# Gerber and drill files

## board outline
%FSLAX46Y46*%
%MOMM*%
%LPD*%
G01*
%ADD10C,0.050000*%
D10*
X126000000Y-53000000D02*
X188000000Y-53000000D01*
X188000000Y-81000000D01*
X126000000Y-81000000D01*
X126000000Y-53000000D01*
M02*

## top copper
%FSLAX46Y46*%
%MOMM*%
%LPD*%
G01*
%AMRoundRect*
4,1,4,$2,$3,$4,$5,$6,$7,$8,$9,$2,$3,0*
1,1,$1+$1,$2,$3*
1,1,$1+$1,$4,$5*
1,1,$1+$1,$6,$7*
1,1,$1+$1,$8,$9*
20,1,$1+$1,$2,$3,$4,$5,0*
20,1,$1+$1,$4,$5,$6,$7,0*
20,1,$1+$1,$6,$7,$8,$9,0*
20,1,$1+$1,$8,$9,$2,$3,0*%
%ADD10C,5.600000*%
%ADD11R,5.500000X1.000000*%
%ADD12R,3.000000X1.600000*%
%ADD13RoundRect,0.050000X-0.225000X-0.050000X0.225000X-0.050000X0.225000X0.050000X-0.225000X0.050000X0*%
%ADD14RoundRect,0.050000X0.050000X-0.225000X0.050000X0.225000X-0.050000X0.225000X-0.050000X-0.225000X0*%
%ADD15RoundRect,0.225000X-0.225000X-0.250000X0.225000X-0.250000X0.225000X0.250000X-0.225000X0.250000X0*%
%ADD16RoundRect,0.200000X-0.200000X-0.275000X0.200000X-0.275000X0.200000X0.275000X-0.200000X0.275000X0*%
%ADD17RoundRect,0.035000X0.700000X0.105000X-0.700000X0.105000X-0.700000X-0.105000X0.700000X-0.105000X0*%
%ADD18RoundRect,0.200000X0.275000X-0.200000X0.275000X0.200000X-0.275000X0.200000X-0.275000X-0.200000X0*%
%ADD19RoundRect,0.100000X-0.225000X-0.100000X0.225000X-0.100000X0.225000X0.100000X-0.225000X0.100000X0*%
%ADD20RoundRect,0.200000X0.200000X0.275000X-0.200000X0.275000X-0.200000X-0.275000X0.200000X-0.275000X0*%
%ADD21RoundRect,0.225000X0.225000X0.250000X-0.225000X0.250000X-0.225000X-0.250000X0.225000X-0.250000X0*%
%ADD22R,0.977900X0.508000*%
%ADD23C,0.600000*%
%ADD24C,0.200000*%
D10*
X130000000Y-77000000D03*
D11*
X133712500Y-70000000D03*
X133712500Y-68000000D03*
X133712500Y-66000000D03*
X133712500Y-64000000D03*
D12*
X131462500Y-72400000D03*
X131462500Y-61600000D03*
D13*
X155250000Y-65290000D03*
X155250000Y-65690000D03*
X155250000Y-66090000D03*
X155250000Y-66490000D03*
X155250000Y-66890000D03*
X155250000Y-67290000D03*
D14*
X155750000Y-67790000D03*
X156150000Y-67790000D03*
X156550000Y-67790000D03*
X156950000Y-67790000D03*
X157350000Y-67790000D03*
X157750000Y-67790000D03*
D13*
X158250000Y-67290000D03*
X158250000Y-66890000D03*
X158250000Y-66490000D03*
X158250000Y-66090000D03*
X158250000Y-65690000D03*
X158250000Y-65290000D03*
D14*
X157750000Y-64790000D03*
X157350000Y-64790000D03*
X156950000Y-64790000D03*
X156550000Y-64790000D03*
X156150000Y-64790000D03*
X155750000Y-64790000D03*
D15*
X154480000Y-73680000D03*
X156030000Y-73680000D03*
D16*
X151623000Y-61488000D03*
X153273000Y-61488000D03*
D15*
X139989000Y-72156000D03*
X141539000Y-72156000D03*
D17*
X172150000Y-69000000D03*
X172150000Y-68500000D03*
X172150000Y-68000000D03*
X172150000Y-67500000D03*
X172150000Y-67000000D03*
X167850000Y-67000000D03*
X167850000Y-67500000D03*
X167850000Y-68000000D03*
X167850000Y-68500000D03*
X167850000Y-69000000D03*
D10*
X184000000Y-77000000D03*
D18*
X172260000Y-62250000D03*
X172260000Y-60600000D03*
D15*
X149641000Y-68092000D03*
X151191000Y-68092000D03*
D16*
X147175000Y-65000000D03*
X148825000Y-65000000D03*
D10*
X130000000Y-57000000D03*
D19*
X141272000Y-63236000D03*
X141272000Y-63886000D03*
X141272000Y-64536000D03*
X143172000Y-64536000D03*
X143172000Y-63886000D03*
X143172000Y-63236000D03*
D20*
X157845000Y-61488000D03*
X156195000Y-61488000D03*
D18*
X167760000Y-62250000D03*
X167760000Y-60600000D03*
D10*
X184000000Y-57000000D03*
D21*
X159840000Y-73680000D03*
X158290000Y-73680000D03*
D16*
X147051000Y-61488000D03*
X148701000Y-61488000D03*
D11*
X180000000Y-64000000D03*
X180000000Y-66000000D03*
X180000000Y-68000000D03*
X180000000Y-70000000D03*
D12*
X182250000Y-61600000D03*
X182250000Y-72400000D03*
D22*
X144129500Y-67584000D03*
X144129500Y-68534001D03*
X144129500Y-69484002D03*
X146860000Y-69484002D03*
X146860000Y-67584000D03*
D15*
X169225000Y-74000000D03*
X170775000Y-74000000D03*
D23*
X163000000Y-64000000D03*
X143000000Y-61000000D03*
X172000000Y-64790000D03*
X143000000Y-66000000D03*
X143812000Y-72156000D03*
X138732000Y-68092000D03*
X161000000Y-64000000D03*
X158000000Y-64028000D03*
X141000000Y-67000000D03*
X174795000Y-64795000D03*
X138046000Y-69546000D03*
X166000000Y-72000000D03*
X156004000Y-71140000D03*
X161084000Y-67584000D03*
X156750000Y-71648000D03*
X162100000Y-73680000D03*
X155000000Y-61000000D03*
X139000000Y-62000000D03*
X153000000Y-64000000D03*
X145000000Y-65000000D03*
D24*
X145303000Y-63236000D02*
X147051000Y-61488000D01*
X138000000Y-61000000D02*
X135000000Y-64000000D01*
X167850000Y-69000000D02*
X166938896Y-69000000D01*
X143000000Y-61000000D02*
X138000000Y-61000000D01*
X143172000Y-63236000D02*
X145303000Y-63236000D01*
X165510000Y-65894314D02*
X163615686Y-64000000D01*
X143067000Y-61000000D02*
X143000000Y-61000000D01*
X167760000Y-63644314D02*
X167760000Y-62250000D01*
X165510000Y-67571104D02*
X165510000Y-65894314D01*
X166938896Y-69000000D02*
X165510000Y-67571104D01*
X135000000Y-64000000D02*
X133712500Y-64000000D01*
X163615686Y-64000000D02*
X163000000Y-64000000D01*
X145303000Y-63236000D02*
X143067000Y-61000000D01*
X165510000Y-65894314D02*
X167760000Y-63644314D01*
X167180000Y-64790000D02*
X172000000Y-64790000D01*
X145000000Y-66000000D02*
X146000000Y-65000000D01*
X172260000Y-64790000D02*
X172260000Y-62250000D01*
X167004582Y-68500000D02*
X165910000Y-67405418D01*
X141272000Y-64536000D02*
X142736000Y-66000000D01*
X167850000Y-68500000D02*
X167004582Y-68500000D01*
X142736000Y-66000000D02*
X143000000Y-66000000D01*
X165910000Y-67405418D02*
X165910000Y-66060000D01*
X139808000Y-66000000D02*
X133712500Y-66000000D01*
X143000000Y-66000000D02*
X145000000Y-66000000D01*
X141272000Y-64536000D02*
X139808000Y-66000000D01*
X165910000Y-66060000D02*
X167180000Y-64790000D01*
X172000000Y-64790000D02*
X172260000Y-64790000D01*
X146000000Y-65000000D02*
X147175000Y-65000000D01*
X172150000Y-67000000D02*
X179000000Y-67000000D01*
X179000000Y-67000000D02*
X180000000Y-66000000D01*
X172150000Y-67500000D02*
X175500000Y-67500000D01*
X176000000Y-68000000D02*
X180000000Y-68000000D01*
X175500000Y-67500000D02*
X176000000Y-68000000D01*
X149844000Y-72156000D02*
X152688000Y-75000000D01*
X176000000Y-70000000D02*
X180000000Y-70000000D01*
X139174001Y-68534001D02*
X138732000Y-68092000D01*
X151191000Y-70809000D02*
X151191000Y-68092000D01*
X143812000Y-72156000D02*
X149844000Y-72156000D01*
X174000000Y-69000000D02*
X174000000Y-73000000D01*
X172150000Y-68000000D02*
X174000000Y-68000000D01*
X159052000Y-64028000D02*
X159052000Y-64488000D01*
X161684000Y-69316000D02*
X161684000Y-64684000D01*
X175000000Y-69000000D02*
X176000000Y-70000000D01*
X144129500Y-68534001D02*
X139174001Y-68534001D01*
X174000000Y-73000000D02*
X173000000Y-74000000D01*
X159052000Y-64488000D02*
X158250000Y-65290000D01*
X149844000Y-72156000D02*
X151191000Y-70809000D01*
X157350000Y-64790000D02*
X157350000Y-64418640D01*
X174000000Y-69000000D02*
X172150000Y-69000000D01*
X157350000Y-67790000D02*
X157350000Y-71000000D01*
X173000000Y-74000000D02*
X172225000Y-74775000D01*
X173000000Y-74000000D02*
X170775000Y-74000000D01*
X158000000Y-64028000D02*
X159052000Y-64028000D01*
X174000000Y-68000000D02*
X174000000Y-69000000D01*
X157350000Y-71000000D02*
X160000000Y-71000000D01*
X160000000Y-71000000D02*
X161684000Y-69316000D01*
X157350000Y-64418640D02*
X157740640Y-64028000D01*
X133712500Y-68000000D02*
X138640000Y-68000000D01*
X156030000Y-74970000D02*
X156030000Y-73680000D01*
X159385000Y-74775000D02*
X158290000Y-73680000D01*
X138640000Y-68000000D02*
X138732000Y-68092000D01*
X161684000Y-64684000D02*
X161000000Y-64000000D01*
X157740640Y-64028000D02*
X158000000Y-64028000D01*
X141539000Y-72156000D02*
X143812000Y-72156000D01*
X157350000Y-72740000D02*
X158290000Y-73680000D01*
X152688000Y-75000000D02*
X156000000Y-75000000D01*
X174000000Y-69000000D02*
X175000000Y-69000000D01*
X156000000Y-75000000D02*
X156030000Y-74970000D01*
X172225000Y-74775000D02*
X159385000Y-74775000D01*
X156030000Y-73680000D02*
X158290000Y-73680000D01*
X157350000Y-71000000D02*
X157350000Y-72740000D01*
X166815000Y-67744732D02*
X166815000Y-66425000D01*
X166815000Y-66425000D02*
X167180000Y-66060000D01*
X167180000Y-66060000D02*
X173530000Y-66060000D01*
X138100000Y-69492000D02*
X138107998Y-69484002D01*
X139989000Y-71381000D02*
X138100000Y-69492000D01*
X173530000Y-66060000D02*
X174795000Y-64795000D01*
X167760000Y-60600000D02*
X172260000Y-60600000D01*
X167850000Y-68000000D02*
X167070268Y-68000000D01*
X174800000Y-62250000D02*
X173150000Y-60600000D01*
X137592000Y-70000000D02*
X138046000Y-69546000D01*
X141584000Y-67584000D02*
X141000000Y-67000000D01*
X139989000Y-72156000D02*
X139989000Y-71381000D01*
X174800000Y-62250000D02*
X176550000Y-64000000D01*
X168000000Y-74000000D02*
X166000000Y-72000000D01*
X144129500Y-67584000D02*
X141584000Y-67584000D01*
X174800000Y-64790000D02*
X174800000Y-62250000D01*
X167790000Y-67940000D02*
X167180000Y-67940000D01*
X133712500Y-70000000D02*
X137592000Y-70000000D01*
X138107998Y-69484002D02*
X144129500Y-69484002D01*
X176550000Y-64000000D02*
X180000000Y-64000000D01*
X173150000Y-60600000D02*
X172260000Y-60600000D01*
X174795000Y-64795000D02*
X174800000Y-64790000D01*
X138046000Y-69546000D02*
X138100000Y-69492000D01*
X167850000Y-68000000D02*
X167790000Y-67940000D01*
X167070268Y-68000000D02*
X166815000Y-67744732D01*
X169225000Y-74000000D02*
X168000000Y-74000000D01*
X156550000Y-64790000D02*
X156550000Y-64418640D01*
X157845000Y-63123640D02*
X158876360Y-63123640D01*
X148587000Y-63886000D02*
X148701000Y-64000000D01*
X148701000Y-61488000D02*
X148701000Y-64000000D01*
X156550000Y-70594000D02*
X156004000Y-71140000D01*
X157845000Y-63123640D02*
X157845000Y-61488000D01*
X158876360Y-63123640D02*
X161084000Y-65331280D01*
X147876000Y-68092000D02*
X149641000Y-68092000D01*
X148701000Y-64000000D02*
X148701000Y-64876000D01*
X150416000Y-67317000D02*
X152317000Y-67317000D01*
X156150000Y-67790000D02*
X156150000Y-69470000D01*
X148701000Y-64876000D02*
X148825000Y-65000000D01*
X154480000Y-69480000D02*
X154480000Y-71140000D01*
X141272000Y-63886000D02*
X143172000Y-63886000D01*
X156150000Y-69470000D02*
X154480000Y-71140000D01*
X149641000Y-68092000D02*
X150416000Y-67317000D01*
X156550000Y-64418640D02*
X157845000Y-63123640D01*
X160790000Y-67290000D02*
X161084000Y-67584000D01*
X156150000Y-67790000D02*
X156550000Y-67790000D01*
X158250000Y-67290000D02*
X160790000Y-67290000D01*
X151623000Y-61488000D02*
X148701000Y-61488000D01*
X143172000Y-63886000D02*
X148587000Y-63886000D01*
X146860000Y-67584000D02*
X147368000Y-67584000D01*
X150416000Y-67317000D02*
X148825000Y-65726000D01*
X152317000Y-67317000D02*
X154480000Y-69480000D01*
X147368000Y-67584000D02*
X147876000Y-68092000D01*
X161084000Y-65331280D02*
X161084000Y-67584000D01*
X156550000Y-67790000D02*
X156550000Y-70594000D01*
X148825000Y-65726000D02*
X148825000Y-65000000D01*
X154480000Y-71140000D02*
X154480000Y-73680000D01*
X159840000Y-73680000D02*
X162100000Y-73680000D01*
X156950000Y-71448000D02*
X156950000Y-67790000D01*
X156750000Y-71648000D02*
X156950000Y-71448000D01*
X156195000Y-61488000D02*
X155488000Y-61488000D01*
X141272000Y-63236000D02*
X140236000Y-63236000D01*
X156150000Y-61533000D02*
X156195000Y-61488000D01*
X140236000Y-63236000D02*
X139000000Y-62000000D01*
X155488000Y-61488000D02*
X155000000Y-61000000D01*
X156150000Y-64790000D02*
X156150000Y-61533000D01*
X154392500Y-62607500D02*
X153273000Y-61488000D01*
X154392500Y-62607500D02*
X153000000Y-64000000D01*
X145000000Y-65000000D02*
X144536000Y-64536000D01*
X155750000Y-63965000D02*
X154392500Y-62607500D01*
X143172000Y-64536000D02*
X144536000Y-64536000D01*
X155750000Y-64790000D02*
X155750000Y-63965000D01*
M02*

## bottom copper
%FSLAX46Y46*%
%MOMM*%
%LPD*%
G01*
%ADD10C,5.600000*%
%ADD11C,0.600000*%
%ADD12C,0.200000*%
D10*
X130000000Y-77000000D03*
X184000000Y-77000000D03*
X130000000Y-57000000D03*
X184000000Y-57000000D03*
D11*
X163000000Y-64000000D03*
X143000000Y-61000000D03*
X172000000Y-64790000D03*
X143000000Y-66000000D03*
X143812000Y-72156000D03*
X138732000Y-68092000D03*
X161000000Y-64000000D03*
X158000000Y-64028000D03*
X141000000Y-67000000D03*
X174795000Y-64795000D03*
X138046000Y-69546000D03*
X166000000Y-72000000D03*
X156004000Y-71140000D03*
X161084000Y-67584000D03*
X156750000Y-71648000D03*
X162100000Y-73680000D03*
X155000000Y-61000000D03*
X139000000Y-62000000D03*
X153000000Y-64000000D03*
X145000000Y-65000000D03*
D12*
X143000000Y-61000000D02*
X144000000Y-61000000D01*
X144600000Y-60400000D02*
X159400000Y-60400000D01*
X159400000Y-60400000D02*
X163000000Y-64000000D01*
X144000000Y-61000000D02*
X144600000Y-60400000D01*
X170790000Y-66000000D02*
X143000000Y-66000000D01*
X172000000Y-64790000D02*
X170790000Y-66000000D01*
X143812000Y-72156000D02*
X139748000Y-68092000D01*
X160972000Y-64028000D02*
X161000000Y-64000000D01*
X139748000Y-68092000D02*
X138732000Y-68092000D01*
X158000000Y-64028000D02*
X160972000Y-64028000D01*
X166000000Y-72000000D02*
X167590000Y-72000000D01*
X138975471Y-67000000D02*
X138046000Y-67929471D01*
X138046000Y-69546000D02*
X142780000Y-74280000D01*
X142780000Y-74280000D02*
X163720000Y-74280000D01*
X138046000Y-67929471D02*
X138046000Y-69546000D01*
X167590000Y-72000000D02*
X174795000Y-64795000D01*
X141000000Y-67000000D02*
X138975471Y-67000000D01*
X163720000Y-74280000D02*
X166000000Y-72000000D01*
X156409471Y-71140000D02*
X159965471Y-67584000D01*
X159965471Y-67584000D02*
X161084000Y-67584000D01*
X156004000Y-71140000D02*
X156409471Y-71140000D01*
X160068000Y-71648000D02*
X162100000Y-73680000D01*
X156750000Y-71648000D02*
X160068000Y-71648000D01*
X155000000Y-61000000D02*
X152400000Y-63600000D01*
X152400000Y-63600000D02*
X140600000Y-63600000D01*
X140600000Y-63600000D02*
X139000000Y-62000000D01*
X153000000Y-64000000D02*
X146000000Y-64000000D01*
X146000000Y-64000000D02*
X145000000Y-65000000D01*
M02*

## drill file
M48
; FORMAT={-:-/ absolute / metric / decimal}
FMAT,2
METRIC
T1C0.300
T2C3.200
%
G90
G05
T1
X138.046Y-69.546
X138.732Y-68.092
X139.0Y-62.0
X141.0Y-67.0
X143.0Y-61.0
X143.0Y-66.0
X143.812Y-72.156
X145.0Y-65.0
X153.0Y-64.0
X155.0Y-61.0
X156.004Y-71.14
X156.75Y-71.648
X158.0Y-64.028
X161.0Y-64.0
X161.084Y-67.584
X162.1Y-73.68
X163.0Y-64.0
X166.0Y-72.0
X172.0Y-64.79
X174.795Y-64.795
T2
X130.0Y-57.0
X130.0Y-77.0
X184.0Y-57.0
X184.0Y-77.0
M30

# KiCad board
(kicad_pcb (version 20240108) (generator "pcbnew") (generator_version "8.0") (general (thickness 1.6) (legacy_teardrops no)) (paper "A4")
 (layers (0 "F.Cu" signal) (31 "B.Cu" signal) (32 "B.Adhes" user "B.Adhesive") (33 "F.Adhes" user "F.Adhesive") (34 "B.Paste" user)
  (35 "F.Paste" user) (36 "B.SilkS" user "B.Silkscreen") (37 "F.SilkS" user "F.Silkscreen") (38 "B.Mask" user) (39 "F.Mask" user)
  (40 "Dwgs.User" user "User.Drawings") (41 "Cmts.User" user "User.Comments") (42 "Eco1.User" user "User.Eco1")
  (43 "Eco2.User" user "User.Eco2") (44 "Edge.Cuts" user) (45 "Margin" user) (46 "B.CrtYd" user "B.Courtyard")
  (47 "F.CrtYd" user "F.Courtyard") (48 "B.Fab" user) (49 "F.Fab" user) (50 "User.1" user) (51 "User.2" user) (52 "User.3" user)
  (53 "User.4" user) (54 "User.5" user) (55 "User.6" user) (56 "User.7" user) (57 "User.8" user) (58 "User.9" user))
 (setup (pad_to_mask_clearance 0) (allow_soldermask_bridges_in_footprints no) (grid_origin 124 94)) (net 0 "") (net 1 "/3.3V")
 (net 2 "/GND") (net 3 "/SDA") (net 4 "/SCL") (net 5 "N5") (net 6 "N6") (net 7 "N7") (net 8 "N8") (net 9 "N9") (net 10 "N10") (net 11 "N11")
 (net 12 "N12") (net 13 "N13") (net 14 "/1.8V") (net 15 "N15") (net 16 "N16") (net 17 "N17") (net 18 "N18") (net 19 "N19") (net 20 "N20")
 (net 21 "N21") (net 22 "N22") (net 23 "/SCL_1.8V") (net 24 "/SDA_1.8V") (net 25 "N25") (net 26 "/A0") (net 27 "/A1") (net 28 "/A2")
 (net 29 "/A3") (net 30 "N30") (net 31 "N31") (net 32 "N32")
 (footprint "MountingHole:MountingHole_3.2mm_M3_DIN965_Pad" (layer "F.Cu") (at 130 77)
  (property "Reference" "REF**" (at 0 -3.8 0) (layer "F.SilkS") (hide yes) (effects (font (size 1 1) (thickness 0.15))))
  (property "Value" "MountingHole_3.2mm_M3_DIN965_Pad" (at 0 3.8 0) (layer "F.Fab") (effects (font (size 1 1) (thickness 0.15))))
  (pad "1" thru_hole circle (at 0 0) (size 5.6 5.6) (drill 3.2) (layers "*.Cu" "*.Mask") (remove_unused_layers no)))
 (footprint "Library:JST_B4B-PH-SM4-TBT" (layer "F.Cu") (at 131.4625 67 90)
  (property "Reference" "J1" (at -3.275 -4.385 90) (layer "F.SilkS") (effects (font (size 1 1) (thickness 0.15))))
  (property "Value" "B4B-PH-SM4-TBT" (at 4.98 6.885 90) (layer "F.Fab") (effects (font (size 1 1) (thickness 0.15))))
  (pad "1" smd rect (at -3 2.25 90) (size 1 5.5) (layers "F.Cu" "F.Paste" "F.Mask") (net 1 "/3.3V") (solder_mask_margin 0.102))
  (pad "2" smd rect (at -1 2.25 90) (size 1 5.5) (layers "F.Cu" "F.Paste" "F.Mask") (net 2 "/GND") (solder_mask_margin 0.102))
  (pad "3" smd rect (at 1 2.25 90) (size 1 5.5) (layers "F.Cu" "F.Paste" "F.Mask") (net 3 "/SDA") (solder_mask_margin 0.102))
  (pad "4" smd rect (at 3 2.25 90) (size 1 5.5) (layers "F.Cu" "F.Paste" "F.Mask") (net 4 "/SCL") (solder_mask_margin 0.102))
  (pad "SH1" smd rect (at -5.4 0 90) (size 1.6 3) (layers "F.Cu" "F.Paste" "F.Mask") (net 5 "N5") (solder_mask_margin 0.102))
  (pad "SH2" smd rect (at 5.4 0 90) (size 1.6 3) (layers "F.Cu" "F.Paste" "F.Mask") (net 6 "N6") (solder_mask_margin 0.102)))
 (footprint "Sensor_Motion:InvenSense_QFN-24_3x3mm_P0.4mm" (layer "F.Cu") (at 156.75 66.29)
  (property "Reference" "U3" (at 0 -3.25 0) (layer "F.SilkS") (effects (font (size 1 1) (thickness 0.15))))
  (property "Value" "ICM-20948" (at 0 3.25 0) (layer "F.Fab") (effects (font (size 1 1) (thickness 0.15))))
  (pad "1" smd roundrect (at -1.5 -1) (size 0.55 0.2) (layers "F.Cu" "F.Paste" "F.Mask") (roundrect_rratio 0.25) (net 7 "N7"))
  (pad "2" smd roundrect (at -1.5 -0.6) (size 0.55 0.2) (layers "F.Cu" "F.Paste" "F.Mask") (roundrect_rratio 0.25) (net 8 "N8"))
  (pad "3" smd roundrect (at -1.5 -0.2) (size 0.55 0.2) (layers "F.Cu" "F.Paste" "F.Mask") (roundrect_rratio 0.25) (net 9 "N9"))
  (pad "4" smd roundrect (at -1.5 0.2) (size 0.55 0.2) (layers "F.Cu" "F.Paste" "F.Mask") (roundrect_rratio 0.25) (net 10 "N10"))
  (pad "5" smd roundrect (at -1.5 0.6) (size 0.55 0.2) (layers "F.Cu" "F.Paste" "F.Mask") (roundrect_rratio 0.25) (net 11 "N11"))
  (pad "6" smd roundrect (at -1.5 1) (size 0.55 0.2) (layers "F.Cu" "F.Paste" "F.Mask") (roundrect_rratio 0.25) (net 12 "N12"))
  (pad "7" smd roundrect (at -1 1.5 90) (size 0.55 0.2) (layers "F.Cu" "F.Paste" "F.Mask") (roundrect_rratio 0.25) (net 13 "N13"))
  (pad "8" smd roundrect (at -0.6 1.5 90) (size 0.55 0.2) (layers "F.Cu" "F.Paste" "F.Mask") (roundrect_rratio 0.25) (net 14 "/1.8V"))
  (pad "9" smd roundrect (at -0.2 1.5 90) (size 0.55 0.2) (layers "F.Cu" "F.Paste" "F.Mask") (roundrect_rratio 0.25) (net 14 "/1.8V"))
  (pad "10" smd roundrect (at 0.2 1.5 90) (size 0.55 0.2) (layers "F.Cu" "F.Paste" "F.Mask") (roundrect_rratio 0.25) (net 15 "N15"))
  (pad "11" smd roundrect (at 0.6 1.5 90) (size 0.55 0.2) (layers "F.Cu" "F.Paste" "F.Mask") (roundrect_rratio 0.25) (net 2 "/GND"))
  (pad "12" smd roundrect (at 1 1.5 90) (size 0.55 0.2) (layers "F.Cu" "F.Paste" "F.Mask") (roundrect_rratio 0.25) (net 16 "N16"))
  (pad "13" smd roundrect (at 1.5 1) (size 0.55 0.2) (layers "F.Cu" "F.Paste" "F.Mask") (roundrect_rratio 0.25) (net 14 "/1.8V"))
  (pad "14" smd roundrect (at 1.5 0.6) (size 0.55 0.2) (layers "F.Cu" "F.Paste" "F.Mask") (roundrect_rratio 0.25) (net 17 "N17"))
  (pad "15" smd roundrect (at 1.5 0.2) (size 0.55 0.2) (layers "F.Cu" "F.Paste" "F.Mask") (roundrect_rratio 0.25) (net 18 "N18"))
  (pad "16" smd roundrect (at 1.5 -0.2) (size 0.55 0.2) (layers "F.Cu" "F.Paste" "F.Mask") (roundrect_rratio 0.25) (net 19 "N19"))
  (pad "17" smd roundrect (at 1.5 -0.6) (size 0.55 0.2) (layers "F.Cu" "F.Paste" "F.Mask") (roundrect_rratio 0.25) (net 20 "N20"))
  (pad "18" smd roundrect (at 1.5 -1) (size 0.55 0.2) (layers "F.Cu" "F.Paste" "F.Mask") (roundrect_rratio 0.25) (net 2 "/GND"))
  (pad "19" smd roundrect (at 1 -1.5 90) (size 0.55 0.2) (layers "F.Cu" "F.Paste" "F.Mask") (roundrect_rratio 0.25) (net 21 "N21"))
  (pad "20" smd roundrect (at 0.6 -1.5 90) (size 0.55 0.2) (layers "F.Cu" "F.Paste" "F.Mask") (roundrect_rratio 0.25) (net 2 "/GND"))
  (pad "21" smd roundrect (at 0.2 -1.5 90) (size 0.55 0.2) (layers "F.Cu" "F.Paste" "F.Mask") (roundrect_rratio 0.25) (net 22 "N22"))
  (pad "22" smd roundrect (at -0.2 -1.5 90) (size 0.55 0.2) (layers "F.Cu" "F.Paste" "F.Mask") (roundrect_rratio 0.25) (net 14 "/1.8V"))
  (pad "23" smd roundrect (at -0.6 -1.5 90) (size 0.55 0.2) (layers "F.Cu" "F.Paste" "F.Mask") (roundrect_rratio 0.25) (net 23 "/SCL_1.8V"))
  (pad "24" smd roundrect (at -1 -1.5 90) (size 0.55 0.2) (layers "F.Cu" "F.Paste" "F.Mask") (roundrect_rratio 0.25) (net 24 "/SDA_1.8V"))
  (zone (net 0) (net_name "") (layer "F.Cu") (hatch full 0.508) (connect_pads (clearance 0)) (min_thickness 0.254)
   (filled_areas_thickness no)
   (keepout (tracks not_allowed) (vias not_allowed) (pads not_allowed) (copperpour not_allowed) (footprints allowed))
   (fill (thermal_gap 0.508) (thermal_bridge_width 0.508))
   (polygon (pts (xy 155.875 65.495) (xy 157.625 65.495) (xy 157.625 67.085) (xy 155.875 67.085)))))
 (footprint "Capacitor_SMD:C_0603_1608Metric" (layer "F.Cu") (at 155.255 73.68)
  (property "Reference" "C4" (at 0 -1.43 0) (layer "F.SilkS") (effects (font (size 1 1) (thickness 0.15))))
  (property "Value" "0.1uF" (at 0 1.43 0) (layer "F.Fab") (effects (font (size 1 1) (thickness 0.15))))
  (pad "1" smd roundrect (at -0.775 0) (size 0.9 0.95) (layers "F.Cu" "F.Paste" "F.Mask") (roundrect_rratio 0.25) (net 14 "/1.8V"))
  (pad "2" smd roundrect (at 0.775 0) (size 0.9 0.95) (layers "F.Cu" "F.Paste" "F.Mask") (roundrect_rratio 0.25) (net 2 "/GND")))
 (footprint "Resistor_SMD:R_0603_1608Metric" (layer "F.Cu") (at 152.448 61.488)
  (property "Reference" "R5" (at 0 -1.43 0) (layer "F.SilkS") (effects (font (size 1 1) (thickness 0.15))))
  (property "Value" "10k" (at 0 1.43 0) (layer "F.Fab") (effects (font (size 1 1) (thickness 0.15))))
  (pad "1" smd roundrect (at -0.825 0) (size 0.8 0.95) (layers "F.Cu" "F.Paste" "F.Mask") (roundrect_rratio 0.25) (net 14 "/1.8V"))
  (pad "2" smd roundrect (at 0.825 0) (size 0.8 0.95) (layers "F.Cu" "F.Paste" "F.Mask") (roundrect_rratio 0.25) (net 24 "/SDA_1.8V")))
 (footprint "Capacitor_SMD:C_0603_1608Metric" (layer "F.Cu") (at 140.764 72.156)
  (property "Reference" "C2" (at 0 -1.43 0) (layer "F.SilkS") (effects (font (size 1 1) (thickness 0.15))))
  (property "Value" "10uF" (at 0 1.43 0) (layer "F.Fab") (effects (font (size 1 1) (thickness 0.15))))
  (pad "1" smd roundrect (at -0.775 0) (size 0.9 0.95) (layers "F.Cu" "F.Paste" "F.Mask") (roundrect_rratio 0.25) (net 1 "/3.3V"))
  (pad "2" smd roundrect (at 0.775 0) (size 0.9 0.95) (layers "F.Cu" "F.Paste" "F.Mask") (roundrect_rratio 0.25) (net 2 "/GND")))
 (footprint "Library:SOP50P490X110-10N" (layer "F.Cu") (at 170 68 180)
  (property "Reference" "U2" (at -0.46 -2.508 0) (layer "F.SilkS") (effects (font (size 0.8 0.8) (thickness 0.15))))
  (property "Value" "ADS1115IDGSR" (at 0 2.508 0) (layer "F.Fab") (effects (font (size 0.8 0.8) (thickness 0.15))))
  (pad "1" smd roundrect (at -2.15 -1 180) (size 1.47 0.28) (layers "F.Cu" "F.Paste" "F.Mask") (roundrect_rratio 0.125) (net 2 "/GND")
   (solder_mask_margin 0.102))
  (pad "2" smd roundrect (at -2.15 -0.5 180) (size 1.47 0.28) (layers "F.Cu" "F.Paste" "F.Mask") (roundrect_rratio 0.125) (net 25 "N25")
   (solder_mask_margin 0.102))
  (pad "3" smd roundrect (at -2.15 0 180) (size 1.47 0.28) (layers "F.Cu" "F.Paste" "F.Mask") (roundrect_rratio 0.125) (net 2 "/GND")
   (solder_mask_margin 0.102))
  (pad "4" smd roundrect (at -2.15 0.5 180) (size 1.47 0.28) (layers "F.Cu" "F.Paste" "F.Mask") (roundrect_rratio 0.125) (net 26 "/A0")
   (solder_mask_margin 0.102))
  (pad "5" smd roundrect (at -2.15 1 180) (size 1.47 0.28) (layers "F.Cu" "F.Paste" "F.Mask") (roundrect_rratio 0.125) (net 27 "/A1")
   (solder_mask_margin 0.102))
  (pad "6" smd roundrect (at 2.15 1 180) (size 1.47 0.28) (layers "F.Cu" "F.Paste" "F.Mask") (roundrect_rratio 0.125) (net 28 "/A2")
   (solder_mask_margin 0.102))
  (pad "7" smd roundrect (at 2.15 0.5 180) (size 1.47 0.28) (layers "F.Cu" "F.Paste" "F.Mask") (roundrect_rratio 0.125) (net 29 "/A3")
   (solder_mask_margin 0.102))
  (pad "8" smd roundrect (at 2.15 0 180) (size 1.47 0.28) (layers "F.Cu" "F.Paste" "F.Mask") (roundrect_rratio 0.125) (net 1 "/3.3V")
   (solder_mask_margin 0.102))
  (pad "9" smd roundrect (at 2.15 -0.5 180) (size 1.47 0.28) (layers "F.Cu" "F.Paste" "F.Mask") (roundrect_rratio 0.125) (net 3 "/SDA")
   (solder_mask_margin 0.102))
  (pad "10" smd roundrect (at 2.15 -1 180) (size 1.47 0.28) (layers "F.Cu" "F.Paste" "F.Mask") (roundrect_rratio 0.125) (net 4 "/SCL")
   (solder_mask_margin 0.102)))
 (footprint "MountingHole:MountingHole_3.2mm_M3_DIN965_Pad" (layer "F.Cu") (at 184 77)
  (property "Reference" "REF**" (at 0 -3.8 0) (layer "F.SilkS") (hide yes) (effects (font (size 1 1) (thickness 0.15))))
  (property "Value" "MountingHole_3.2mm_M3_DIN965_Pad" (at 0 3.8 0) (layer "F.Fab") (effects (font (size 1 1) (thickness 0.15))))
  (pad "1" thru_hole circle (at 0 0) (size 5.6 5.6) (drill 3.2) (layers "*.Cu" "*.Mask") (remove_unused_layers no)))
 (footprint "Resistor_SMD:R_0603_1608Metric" (layer "F.Cu") (at 172.26 61.425 90)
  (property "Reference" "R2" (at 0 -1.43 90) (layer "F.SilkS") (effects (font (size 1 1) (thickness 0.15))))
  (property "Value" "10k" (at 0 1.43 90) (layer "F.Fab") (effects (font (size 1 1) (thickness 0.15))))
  (pad "1" smd roundrect (at -0.825 0 90) (size 0.8 0.95) (layers "F.Cu" "F.Paste" "F.Mask") (roundrect_rratio 0.25) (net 3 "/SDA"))
  (pad "2" smd roundrect (at 0.825 0 90) (size 0.8 0.95) (layers "F.Cu" "F.Paste" "F.Mask") (roundrect_rratio 0.25) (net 1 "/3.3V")))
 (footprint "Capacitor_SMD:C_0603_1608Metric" (layer "F.Cu") (at 150.416 68.092)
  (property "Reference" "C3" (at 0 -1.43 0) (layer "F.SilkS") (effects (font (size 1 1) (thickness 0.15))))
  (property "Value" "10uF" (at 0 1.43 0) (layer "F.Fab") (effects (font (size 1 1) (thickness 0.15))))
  (pad "1" smd roundrect (at -0.775 0) (size 0.9 0.95) (layers "F.Cu" "F.Paste" "F.Mask") (roundrect_rratio 0.25) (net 14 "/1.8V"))
  (pad "2" smd roundrect (at 0.775 0) (size 0.9 0.95) (layers "F.Cu" "F.Paste" "F.Mask") (roundrect_rratio 0.25) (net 2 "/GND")))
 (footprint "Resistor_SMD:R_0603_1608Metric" (layer "F.Cu") (at 148 65)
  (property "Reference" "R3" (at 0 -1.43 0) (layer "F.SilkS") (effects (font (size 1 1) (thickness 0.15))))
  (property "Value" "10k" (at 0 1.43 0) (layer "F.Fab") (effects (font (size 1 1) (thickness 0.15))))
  (pad "1" smd roundrect (at -0.825 0) (size 0.8 0.95) (layers "F.Cu" "F.Paste" "F.Mask") (roundrect_rratio 0.25) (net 3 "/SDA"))
  (pad "2" smd roundrect (at 0.825 0) (size 0.8 0.95) (layers "F.Cu" "F.Paste" "F.Mask") (roundrect_rratio 0.25) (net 14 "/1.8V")))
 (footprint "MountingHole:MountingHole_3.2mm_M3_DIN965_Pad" (layer "F.Cu") (at 130 57)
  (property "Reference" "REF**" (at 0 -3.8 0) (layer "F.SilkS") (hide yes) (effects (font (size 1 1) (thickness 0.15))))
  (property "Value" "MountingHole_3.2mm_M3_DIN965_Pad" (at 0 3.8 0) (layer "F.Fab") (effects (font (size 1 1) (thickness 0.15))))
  (pad "1" thru_hole circle (at 0 0) (size 5.6 5.6) (drill 3.2) (layers "*.Cu" "*.Mask") (remove_unused_layers no)))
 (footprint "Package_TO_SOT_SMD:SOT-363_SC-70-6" (layer "F.Cu") (at 142.222 63.886)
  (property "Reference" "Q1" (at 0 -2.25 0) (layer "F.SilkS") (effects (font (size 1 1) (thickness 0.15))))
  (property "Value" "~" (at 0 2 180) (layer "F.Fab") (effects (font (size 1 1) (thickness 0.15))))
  (pad "1" smd roundrect (at -0.95 -0.65) (size 0.65 0.4) (layers "F.Cu" "F.Paste" "F.Mask") (roundrect_rratio 0.25) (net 23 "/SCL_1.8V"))
  (pad "2" smd roundrect (at -0.95 0) (size 0.65 0.4) (layers "F.Cu" "F.Paste" "F.Mask") (roundrect_rratio 0.25) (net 14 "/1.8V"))
  (pad "3" smd roundrect (at -0.95 0.65) (size 0.65 0.4) (layers "F.Cu" "F.Paste" "F.Mask") (roundrect_rratio 0.25) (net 3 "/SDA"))
  (pad "4" smd roundrect (at 0.95 0.65) (size 0.65 0.4) (layers "F.Cu" "F.Paste" "F.Mask") (roundrect_rratio 0.25) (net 24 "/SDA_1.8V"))
  (pad "5" smd roundrect (at 0.95 0) (size 0.65 0.4) (layers "F.Cu" "F.Paste" "F.Mask") (roundrect_rratio 0.25) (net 14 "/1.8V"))
  (pad "6" smd roundrect (at 0.95 -0.65) (size 0.65 0.4) (layers "F.Cu" "F.Paste" "F.Mask") (roundrect_rratio 0.25) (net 4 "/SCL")))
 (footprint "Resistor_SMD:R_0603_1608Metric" (layer "F.Cu") (at 157.02 61.488 180)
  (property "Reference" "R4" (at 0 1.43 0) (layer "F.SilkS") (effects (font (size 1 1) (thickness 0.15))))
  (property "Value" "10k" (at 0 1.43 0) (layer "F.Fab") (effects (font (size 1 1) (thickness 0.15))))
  (pad "1" smd roundrect (at -0.825 0 180) (size 0.8 0.95) (layers "F.Cu" "F.Paste" "F.Mask") (roundrect_rratio 0.25) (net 14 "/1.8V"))
  (pad "2" smd roundrect (at 0.825 0 180) (size 0.8 0.95) (layers "F.Cu" "F.Paste" "F.Mask") (roundrect_rratio 0.25) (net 23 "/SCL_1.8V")))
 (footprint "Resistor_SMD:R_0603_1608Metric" (layer "F.Cu") (at 167.76 61.425 90)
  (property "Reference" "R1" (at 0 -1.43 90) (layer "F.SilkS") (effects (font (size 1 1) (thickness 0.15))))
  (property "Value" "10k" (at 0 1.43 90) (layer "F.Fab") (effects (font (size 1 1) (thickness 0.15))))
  (pad "1" smd roundrect (at -0.825 0 90) (size 0.8 0.95) (layers "F.Cu" "F.Paste" "F.Mask") (roundrect_rratio 0.25) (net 4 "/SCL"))
  (pad "2" smd roundrect (at 0.825 0 90) (size 0.8 0.95) (layers "F.Cu" "F.Paste" "F.Mask") (roundrect_rratio 0.25) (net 1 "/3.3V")))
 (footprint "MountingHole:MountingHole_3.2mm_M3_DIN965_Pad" (layer "F.Cu") (at 184 57)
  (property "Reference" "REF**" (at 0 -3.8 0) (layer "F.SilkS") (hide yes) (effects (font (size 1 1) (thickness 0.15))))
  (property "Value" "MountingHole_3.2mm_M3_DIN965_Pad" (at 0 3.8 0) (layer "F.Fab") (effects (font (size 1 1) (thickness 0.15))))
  (pad "1" thru_hole circle (at 0 0) (size 5.6 5.6) (drill 3.2) (layers "*.Cu" "*.Mask") (remove_unused_layers no)))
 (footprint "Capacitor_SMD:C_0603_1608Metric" (layer "F.Cu") (at 159.065 73.68 180)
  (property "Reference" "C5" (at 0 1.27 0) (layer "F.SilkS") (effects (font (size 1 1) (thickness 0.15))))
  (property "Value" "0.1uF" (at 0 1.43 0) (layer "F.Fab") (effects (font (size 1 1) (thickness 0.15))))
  (pad "1" smd roundrect (at -0.775 0 180) (size 0.9 0.95) (layers "F.Cu" "F.Paste" "F.Mask") (roundrect_rratio 0.25) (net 15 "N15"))
  (pad "2" smd roundrect (at 0.775 0 180) (size 0.9 0.95) (layers "F.Cu" "F.Paste" "F.Mask") (roundrect_rratio 0.25) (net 2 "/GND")))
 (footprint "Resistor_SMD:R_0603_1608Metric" (layer "F.Cu") (at 147.876 61.488)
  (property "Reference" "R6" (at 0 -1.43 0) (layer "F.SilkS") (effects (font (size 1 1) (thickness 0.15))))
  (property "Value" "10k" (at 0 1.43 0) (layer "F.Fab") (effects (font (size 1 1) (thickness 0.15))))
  (pad "1" smd roundrect (at -0.825 0) (size 0.8 0.95) (layers "F.Cu" "F.Paste" "F.Mask") (roundrect_rratio 0.25) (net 4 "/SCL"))
  (pad "2" smd roundrect (at 0.825 0) (size 0.8 0.95) (layers "F.Cu" "F.Paste" "F.Mask") (roundrect_rratio 0.25) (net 14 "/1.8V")))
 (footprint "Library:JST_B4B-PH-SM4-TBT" (layer "F.Cu") (at 182.25 67 -90)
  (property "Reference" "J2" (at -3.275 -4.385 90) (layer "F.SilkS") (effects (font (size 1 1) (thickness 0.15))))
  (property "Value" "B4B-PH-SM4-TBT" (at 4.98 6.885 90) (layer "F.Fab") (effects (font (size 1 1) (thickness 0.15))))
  (pad "1" smd rect (at -3 2.25 270) (size 1 5.5) (layers "F.Cu" "F.Paste" "F.Mask") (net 1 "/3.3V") (solder_mask_margin 0.102))
  (pad "2" smd rect (at -1 2.25 270) (size 1 5.5) (layers "F.Cu" "F.Paste" "F.Mask") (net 27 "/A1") (solder_mask_margin 0.102))
  (pad "3" smd rect (at 1 2.25 270) (size 1 5.5) (layers "F.Cu" "F.Paste" "F.Mask") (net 26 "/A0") (solder_mask_margin 0.102))
  (pad "4" smd rect (at 3 2.25 270) (size 1 5.5) (layers "F.Cu" "F.Paste" "F.Mask") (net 2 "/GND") (solder_mask_margin 0.102))
  (pad "SH1" smd rect (at -5.4 0 270) (size 1.6 3) (layers "F.Cu" "F.Paste" "F.Mask") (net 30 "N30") (solder_mask_margin 0.102))
  (pad "SH2" smd rect (at 5.4 0 270) (size 1.6 3) (layers "F.Cu" "F.Paste" "F.Mask") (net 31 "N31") (solder_mask_margin 0.102)))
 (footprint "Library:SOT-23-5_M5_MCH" (layer "F.Cu") (at 145.49475 68.534001)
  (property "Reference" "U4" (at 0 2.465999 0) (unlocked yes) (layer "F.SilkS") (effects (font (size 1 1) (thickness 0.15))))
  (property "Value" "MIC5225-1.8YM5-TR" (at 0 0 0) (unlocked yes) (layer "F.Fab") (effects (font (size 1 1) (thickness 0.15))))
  (pad "1" smd rect (at -1.36525 -0.950001) (size 0.9779 0.508) (layers "F.Cu" "F.Paste" "F.Mask") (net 1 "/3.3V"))
  (pad "2" smd rect (at -1.36525 0) (size 0.9779 0.508) (layers "F.Cu" "F.Paste" "F.Mask") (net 2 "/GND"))
  (pad "3" smd rect (at -1.36525 0.950001) (size 0.9779 0.508) (layers "F.Cu" "F.Paste" "F.Mask") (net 1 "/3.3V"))
  (pad "4" smd rect (at 1.36525 0.950001) (size 0.9779 0.508) (layers "F.Cu" "F.Paste" "F.Mask") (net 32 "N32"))
  (pad "5" smd rect (at 1.36525 -0.950001) (size 0.9779 0.508) (layers "F.Cu" "F.Paste" "F.Mask") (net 14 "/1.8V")))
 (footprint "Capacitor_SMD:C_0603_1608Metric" (layer "F.Cu") (at 170 74)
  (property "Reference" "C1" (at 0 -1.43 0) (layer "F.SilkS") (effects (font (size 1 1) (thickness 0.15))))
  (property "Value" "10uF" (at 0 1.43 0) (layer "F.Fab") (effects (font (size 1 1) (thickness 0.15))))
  (pad "1" smd roundrect (at -0.775 0) (size 0.9 0.95) (layers "F.Cu" "F.Paste" "F.Mask") (roundrect_rratio 0.25) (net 1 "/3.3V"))
  (pad "2" smd roundrect (at 0.775 0) (size 0.9 0.95) (layers "F.Cu" "F.Paste" "F.Mask") (roundrect_rratio 0.25) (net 2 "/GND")))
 (gr_rect (start 126 53) (end 188 81) (stroke (width 0.05) (type default)) (fill none) (layer "Edge.Cuts"))
 (segment (start 145.303 63.236) (end 147.051 61.488) (width 0.2) (layer "F.Cu") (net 4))
 (segment (start 138 61) (end 135 64) (width 0.2) (layer "F.Cu") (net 4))
 (segment (start 167.85 69) (end 166.938896 69) (width 0.2) (layer "F.Cu") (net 4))
 (segment (start 143 61) (end 138 61) (width 0.2) (layer "F.Cu") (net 4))
 (segment (start 143.172 63.236) (end 145.303 63.236) (width 0.2) (layer "F.Cu") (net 4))
 (segment (start 165.51 65.894314) (end 163.615686 64) (width 0.2) (layer "F.Cu") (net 4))
 (segment (start 143.067 61) (end 143 61) (width 0.2) (layer "F.Cu") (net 4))
 (segment (start 167.76 63.644314) (end 167.76 62.25) (width 0.2) (layer "F.Cu") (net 4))
 (segment (start 165.51 67.571104) (end 165.51 65.894314) (width 0.2) (layer "F.Cu") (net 4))
 (segment (start 166.938896 69) (end 165.51 67.571104) (width 0.2) (layer "F.Cu") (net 4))
 (segment (start 135 64) (end 133.7125 64) (width 0.2) (layer "F.Cu") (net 4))
 (segment (start 163.615686 64) (end 163 64) (width 0.2) (layer "F.Cu") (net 4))
 (segment (start 145.303 63.236) (end 143.067 61) (width 0.2) (layer "F.Cu") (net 4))
 (segment (start 165.51 65.894314) (end 167.76 63.644314) (width 0.2) (layer "F.Cu") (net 4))
 (via (at 163 64) (size 0.6) (drill 0.3) (layers "F.Cu" "B.Cu") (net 4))
 (via (at 143 61) (size 0.6) (drill 0.3) (layers "F.Cu" "B.Cu") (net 4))
 (segment (start 143 61) (end 144 61) (width 0.2) (layer "B.Cu") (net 4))
 (segment (start 144.6 60.4) (end 159.4 60.4) (width 0.2) (layer "B.Cu") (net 4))
 (segment (start 159.4 60.4) (end 163 64) (width 0.2) (layer "B.Cu") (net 4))
 (segment (start 144 61) (end 144.6 60.4) (width 0.2) (layer "B.Cu") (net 4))
 (segment (start 167.18 64.79) (end 172 64.79) (width 0.2) (layer "F.Cu") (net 3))
 (segment (start 145 66) (end 146 65) (width 0.2) (layer "F.Cu") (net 3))
 (segment (start 172.26 64.79) (end 172.26 62.25) (width 0.2) (layer "F.Cu") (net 3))
 (segment (start 167.004582 68.5) (end 165.91 67.405418) (width 0.2) (layer "F.Cu") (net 3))
 (segment (start 141.272 64.536) (end 142.736 66) (width 0.2) (layer "F.Cu") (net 3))
 (segment (start 167.85 68.5) (end 167.004582 68.5) (width 0.2) (layer "F.Cu") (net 3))
 (segment (start 142.736 66) (end 143 66) (width 0.2) (layer "F.Cu") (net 3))
 (segment (start 165.91 67.405418) (end 165.91 66.06) (width 0.2) (layer "F.Cu") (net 3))
 (segment (start 139.808 66) (end 133.7125 66) (width 0.2) (layer "F.Cu") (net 3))
 (segment (start 143 66) (end 145 66) (width 0.2) (layer "F.Cu") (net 3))
 (segment (start 141.272 64.536) (end 139.808 66) (width 0.2) (layer "F.Cu") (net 3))
 (segment (start 165.91 66.06) (end 167.18 64.79) (width 0.2) (layer "F.Cu") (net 3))
 (segment (start 172 64.79) (end 172.26 64.79) (width 0.2) (layer "F.Cu") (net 3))
 (segment (start 146 65) (end 147.175 65) (width 0.2) (layer "F.Cu") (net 3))
 (via (at 172 64.79) (size 0.6) (drill 0.3) (layers "F.Cu" "B.Cu") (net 3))
 (via (at 143 66) (size 0.6) (drill 0.3) (layers "F.Cu" "B.Cu") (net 3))
 (segment (start 170.79 66) (end 143 66) (width 0.2) (layer "B.Cu") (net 3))
 (segment (start 172 64.79) (end 170.79 66) (width 0.2) (layer "B.Cu") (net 3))
 (segment (start 172.15 67) (end 179 67) (width 0.2) (layer "F.Cu") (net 27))
 (segment (start 179 67) (end 180 66) (width 0.2) (layer "F.Cu") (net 27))
 (segment (start 172.15 67.5) (end 175.5 67.5) (width 0.2) (layer "F.Cu") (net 26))
 (segment (start 176 68) (end 180 68) (width 0.2) (layer "F.Cu") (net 26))
 (segment (start 175.5 67.5) (end 176 68) (width 0.2) (layer "F.Cu") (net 26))
 (segment (start 149.844 72.156) (end 152.688 75) (width 0.2) (layer "F.Cu") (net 2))
 (segment (start 176 70) (end 180 70) (width 0.2) (layer "F.Cu") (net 2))
 (segment (start 139.174001 68.534001) (end 138.732 68.092) (width 0.2) (layer "F.Cu") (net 2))
 (segment (start 151.191 70.809) (end 151.191 68.092) (width 0.2) (layer "F.Cu") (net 2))
 (segment (start 143.812 72.156) (end 149.844 72.156) (width 0.2) (layer "F.Cu") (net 2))
 (segment (start 174 69) (end 174 73) (width 0.2) (layer "F.Cu") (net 2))
 (segment (start 172.15 68) (end 174 68) (width 0.2) (layer "F.Cu") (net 2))
 (segment (start 159.052 64.028) (end 159.052 64.488) (width 0.2) (layer "F.Cu") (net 2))
 (segment (start 161.684 69.316) (end 161.684 64.684) (width 0.2) (layer "F.Cu") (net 2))
 (segment (start 175 69) (end 176 70) (width 0.2) (layer "F.Cu") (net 2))
 (segment (start 144.1295 68.534001) (end 139.174001 68.534001) (width 0.2) (layer "F.Cu") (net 2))
 (segment (start 174 73) (end 173 74) (width 0.2) (layer "F.Cu") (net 2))
 (segment (start 159.052 64.488) (end 158.25 65.29) (width 0.2) (layer "F.Cu") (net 2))
 (segment (start 149.844 72.156) (end 151.191 70.809) (width 0.2) (layer "F.Cu") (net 2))
 (segment (start 157.35 64.79) (end 157.35 64.41864) (width 0.2) (layer "F.Cu") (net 2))
 (segment (start 174 69) (end 172.15 69) (width 0.2) (layer "F.Cu") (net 2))
 (segment (start 157.35 67.79) (end 157.35 71) (width 0.2) (layer "F.Cu") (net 2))
 (segment (start 173 74) (end 172.225 74.775) (width 0.2) (layer "F.Cu") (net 2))
 (segment (start 173 74) (end 170.775 74) (width 0.2) (layer "F.Cu") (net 2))
 (segment (start 158 64.028) (end 159.052 64.028) (width 0.2) (layer "F.Cu") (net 2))
 (segment (start 174 68) (end 174 69) (width 0.2) (layer "F.Cu") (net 2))
 (segment (start 157.35 71) (end 160 71) (width 0.2) (layer "F.Cu") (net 2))
 (segment (start 160 71) (end 161.684 69.316) (width 0.2) (layer "F.Cu") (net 2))
 (segment (start 157.35 64.41864) (end 157.74064 64.028) (width 0.2) (layer "F.Cu") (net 2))
 (segment (start 133.7125 68) (end 138.64 68) (width 0.2) (layer "F.Cu") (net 2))
 (segment (start 156.03 74.97) (end 156.03 73.68) (width 0.2) (layer "F.Cu") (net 2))
 (segment (start 159.385 74.775) (end 158.29 73.68) (width 0.2) (layer "F.Cu") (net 2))
 (segment (start 138.64 68) (end 138.732 68.092) (width 0.2) (layer "F.Cu") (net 2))
 (segment (start 161.684 64.684) (end 161 64) (width 0.2) (layer "F.Cu") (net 2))
 (segment (start 157.74064 64.028) (end 158 64.028) (width 0.2) (layer "F.Cu") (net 2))
 (segment (start 141.539 72.156) (end 143.812 72.156) (width 0.2) (layer "F.Cu") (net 2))
 (segment (start 157.35 72.74) (end 158.29 73.68) (width 0.2) (layer "F.Cu") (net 2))
 (segment (start 152.688 75) (end 156 75) (width 0.2) (layer "F.Cu") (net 2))
 (segment (start 174 69) (end 175 69) (width 0.2) (layer "F.Cu") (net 2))
 (segment (start 156 75) (end 156.03 74.97) (width 0.2) (layer "F.Cu") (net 2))
 (segment (start 172.225 74.775) (end 159.385 74.775) (width 0.2) (layer "F.Cu") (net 2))
 (segment (start 156.03 73.68) (end 158.29 73.68) (width 0.2) (layer "F.Cu") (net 2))
 (segment (start 157.35 71) (end 157.35 72.74) (width 0.2) (layer "F.Cu") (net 2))
 (via (at 143.812 72.156) (size 0.6) (drill 0.3) (layers "F.Cu" "B.Cu") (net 2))
 (via (at 138.732 68.092) (size 0.6) (drill 0.3) (layers "F.Cu" "B.Cu") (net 2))
 (via (at 161 64) (size 0.6) (drill 0.3) (layers "F.Cu" "B.Cu") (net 2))
 (via (at 158 64.028) (size 0.6) (drill 0.3) (layers "F.Cu" "B.Cu") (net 2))
 (segment (start 143.812 72.156) (end 139.748 68.092) (width 0.2) (layer "B.Cu") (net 2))
 (segment (start 160.972 64.028) (end 161 64) (width 0.2) (layer "B.Cu") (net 2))
 (segment (start 139.748 68.092) (end 138.732 68.092) (width 0.2) (layer "B.Cu") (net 2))
 (segment (start 158 64.028) (end 160.972 64.028) (width 0.2) (layer "B.Cu") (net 2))
 (segment (start 166.815 67.744732) (end 166.815 66.425) (width 0.2) (layer "F.Cu") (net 1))
 (segment (start 166.815 66.425) (end 167.18 66.06) (width 0.2) (layer "F.Cu") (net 1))
 (segment (start 167.18 66.06) (end 173.53 66.06) (width 0.2) (layer "F.Cu") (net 1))
 (segment (start 138.1 69.492) (end 138.107998 69.484002) (width 0.2) (layer "F.Cu") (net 1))
 (segment (start 139.989 71.381) (end 138.1 69.492) (width 0.2) (layer "F.Cu") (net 1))
 (segment (start 173.53 66.06) (end 174.795 64.795) (width 0.2) (layer "F.Cu") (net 1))
 (segment (start 167.76 60.6) (end 172.26 60.6) (width 0.2) (layer "F.Cu") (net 1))
 (segment (start 167.85 68) (end 167.070268 68) (width 0.2) (layer "F.Cu") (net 1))
 (segment (start 174.8 62.25) (end 173.15 60.6) (width 0.2) (layer "F.Cu") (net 1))
 (segment (start 137.592 70) (end 138.046 69.546) (width 0.2) (layer "F.Cu") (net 1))
 (segment (start 141.584 67.584) (end 141 67) (width 0.2) (layer "F.Cu") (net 1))
 (segment (start 139.989 72.156) (end 139.989 71.381) (width 0.2) (layer "F.Cu") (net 1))
 (segment (start 174.8 62.25) (end 176.55 64) (width 0.2) (layer "F.Cu") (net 1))
 (segment (start 168 74) (end 166 72) (width 0.2) (layer "F.Cu") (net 1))
 (segment (start 144.1295 67.584) (end 141.584 67.584) (width 0.2) (layer "F.Cu") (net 1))
 (segment (start 174.8 64.79) (end 174.8 62.25) (width 0.2) (layer "F.Cu") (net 1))
 (segment (start 167.79 67.94) (end 167.18 67.94) (width 0.2) (layer "F.Cu") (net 1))
 (segment (start 133.7125 70) (end 137.592 70) (width 0.2) (layer "F.Cu") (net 1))
 (segment (start 138.107998 69.484002) (end 144.1295 69.484002) (width 0.2) (layer "F.Cu") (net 1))
 (segment (start 176.55 64) (end 180 64) (width 0.2) (layer "F.Cu") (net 1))
 (segment (start 173.15 60.6) (end 172.26 60.6) (width 0.2) (layer "F.Cu") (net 1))
 (segment (start 174.795 64.795) (end 174.8 64.79) (width 0.2) (layer "F.Cu") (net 1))
 (segment (start 138.046 69.546) (end 138.1 69.492) (width 0.2) (layer "F.Cu") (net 1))
 (segment (start 167.85 68) (end 167.79 67.94) (width 0.2) (layer "F.Cu") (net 1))
 (segment (start 167.070268 68) (end 166.815 67.744732) (width 0.2) (layer "F.Cu") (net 1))
 (segment (start 169.225 74) (end 168 74) (width 0.2) (layer "F.Cu") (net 1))
 (via (at 141 67) (size 0.6) (drill 0.3) (layers "F.Cu" "B.Cu") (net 1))
 (via (at 174.795 64.795) (size 0.6) (drill 0.3) (layers "F.Cu" "B.Cu") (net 1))
 (via (at 138.046 69.546) (size 0.6) (drill 0.3) (layers "F.Cu" "B.Cu") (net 1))
 (via (at 166 72) (size 0.6) (drill 0.3) (layers "F.Cu" "B.Cu") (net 1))
 (segment (start 166 72) (end 167.59 72) (width 0.2) (layer "B.Cu") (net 1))
 (segment (start 138.975471 67) (end 138.046 67.929471) (width 0.2) (layer "B.Cu") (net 1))
 (segment (start 138.046 69.546) (end 142.78 74.28) (width 0.2) (layer "B.Cu") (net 1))
 (segment (start 142.78 74.28) (end 163.72 74.28) (width 0.2) (layer "B.Cu") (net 1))
 (segment (start 138.046 67.929471) (end 138.046 69.546) (width 0.2) (layer "B.Cu") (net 1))
 (segment (start 167.59 72) (end 174.795 64.795) (width 0.2) (layer "B.Cu") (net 1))
 (segment (start 141 67) (end 138.975471 67) (width 0.2) (layer "B.Cu") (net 1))
 (segment (start 163.72 74.28) (end 166 72) (width 0.2) (layer "B.Cu") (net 1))
 (segment (start 156.55 64.79) (end 156.55 64.41864) (width 0.2) (layer "F.Cu") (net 14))
 (segment (start 157.845 63.12364) (end 158.87636 63.12364) (width 0.2) (layer "F.Cu") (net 14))
 (segment (start 148.587 63.886) (end 148.701 64) (width 0.2) (layer "F.Cu") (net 14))
 (segment (start 148.701 61.488) (end 148.701 64) (width 0.2) (layer "F.Cu") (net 14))
 (segment (start 156.55 70.594) (end 156.004 71.14) (width 0.2) (layer "F.Cu") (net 14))
 (segment (start 157.845 63.12364) (end 157.845 61.488) (width 0.2) (layer "F.Cu") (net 14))
 (segment (start 158.87636 63.12364) (end 161.084 65.33128) (width 0.2) (layer "F.Cu") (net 14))
 (segment (start 147.876 68.092) (end 149.641 68.092) (width 0.2) (layer "F.Cu") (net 14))
 (segment (start 148.701 64) (end 148.701 64.876) (width 0.2) (layer "F.Cu") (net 14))
 (segment (start 150.416 67.317) (end 152.317 67.317) (width 0.2) (layer "F.Cu") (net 14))
 (segment (start 156.15 67.79) (end 156.15 69.47) (width 0.2) (layer "F.Cu") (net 14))
 (segment (start 148.701 64.876) (end 148.825 65) (width 0.2) (layer "F.Cu") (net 14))
 (segment (start 154.48 69.48) (end 154.48 71.14) (width 0.2) (layer "F.Cu") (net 14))
 (segment (start 141.272 63.886) (end 143.172 63.886) (width 0.2) (layer "F.Cu") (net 14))
 (segment (start 156.15 69.47) (end 154.48 71.14) (width 0.2) (layer "F.Cu") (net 14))
 (segment (start 149.641 68.092) (end 150.416 67.317) (width 0.2) (layer "F.Cu") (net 14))
 (segment (start 156.55 64.41864) (end 157.845 63.12364) (width 0.2) (layer "F.Cu") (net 14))
 (segment (start 160.79 67.29) (end 161.084 67.584) (width 0.2) (layer "F.Cu") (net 14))
 (segment (start 156.15 67.79) (end 156.55 67.79) (width 0.2) (layer "F.Cu") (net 14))
 (segment (start 158.25 67.29) (end 160.79 67.29) (width 0.2) (layer "F.Cu") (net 14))
 (segment (start 151.623 61.488) (end 148.701 61.488) (width 0.2) (layer "F.Cu") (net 14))
 (segment (start 143.172 63.886) (end 148.587 63.886) (width 0.2) (layer "F.Cu") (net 14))
 (segment (start 146.86 67.584) (end 147.368 67.584) (width 0.2) (layer "F.Cu") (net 14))
 (segment (start 150.416 67.317) (end 148.825 65.726) (width 0.2) (layer "F.Cu") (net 14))
 (segment (start 152.317 67.317) (end 154.48 69.48) (width 0.2) (layer "F.Cu") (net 14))
 (segment (start 147.368 67.584) (end 147.876 68.092) (width 0.2) (layer "F.Cu") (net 14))
 (segment (start 161.084 65.33128) (end 161.084 67.584) (width 0.2) (layer "F.Cu") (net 14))
 (segment (start 156.55 67.79) (end 156.55 70.594) (width 0.2) (layer "F.Cu") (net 14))
 (segment (start 148.825 65.726) (end 148.825 65) (width 0.2) (layer "F.Cu") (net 14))
 (segment (start 154.48 71.14) (end 154.48 73.68) (width 0.2) (layer "F.Cu") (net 14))
 (via (at 156.004 71.14) (size 0.6) (drill 0.3) (layers "F.Cu" "B.Cu") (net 14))
 (via (at 161.084 67.584) (size 0.6) (drill 0.3) (layers "F.Cu" "B.Cu") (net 14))
 (segment (start 156.409471 71.14) (end 159.965471 67.584) (width 0.2) (layer "B.Cu") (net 14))
 (segment (start 159.965471 67.584) (end 161.084 67.584) (width 0.2) (layer "B.Cu") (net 14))
 (segment (start 156.004 71.14) (end 156.409471 71.14) (width 0.2) (layer "B.Cu") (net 14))
 (segment (start 159.84 73.68) (end 162.1 73.68) (width 0.2) (layer "F.Cu") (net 15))
 (segment (start 156.95 71.448) (end 156.95 67.79) (width 0.2) (layer "F.Cu") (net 15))
 (segment (start 156.75 71.648) (end 156.95 71.448) (width 0.2) (layer "F.Cu") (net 15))
 (via (at 156.75 71.648) (size 0.6) (drill 0.3) (layers "F.Cu" "B.Cu") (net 15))
 (via (at 162.1 73.68) (size 0.6) (drill 0.3) (layers "F.Cu" "B.Cu") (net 15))
 (segment (start 160.068 71.648) (end 162.1 73.68) (width 0.2) (layer "B.Cu") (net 15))
 (segment (start 156.75 71.648) (end 160.068 71.648) (width 0.2) (layer "B.Cu") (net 15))
 (segment (start 156.195 61.488) (end 155.488 61.488) (width 0.2) (layer "F.Cu") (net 23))
 (segment (start 141.272 63.236) (end 140.236 63.236) (width 0.2) (layer "F.Cu") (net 23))
 (segment (start 156.15 61.533) (end 156.195 61.488) (width 0.2) (layer "F.Cu") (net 23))
 (segment (start 140.236 63.236) (end 139 62) (width 0.2) (layer "F.Cu") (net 23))
 (segment (start 155.488 61.488) (end 155 61) (width 0.2) (layer "F.Cu") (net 23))
 (segment (start 156.15 64.79) (end 156.15 61.533) (width 0.2) (layer "F.Cu") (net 23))
 (via (at 155 61) (size 0.6) (drill 0.3) (layers "F.Cu" "B.Cu") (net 23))
 (via (at 139 62) (size 0.6) (drill 0.3) (layers "F.Cu" "B.Cu") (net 23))
 (segment (start 155 61) (end 152.4 63.6) (width 0.2) (layer "B.Cu") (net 23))
 (segment (start 152.4 63.6) (end 140.6 63.6) (width 0.2) (layer "B.Cu") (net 23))
 (segment (start 140.6 63.6) (end 139 62) (width 0.2) (layer "B.Cu") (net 23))
 (segment (start 154.3925 62.6075) (end 153.273 61.488) (width 0.2) (layer "F.Cu") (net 24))
 (segment (start 154.3925 62.6075) (end 153 64) (width 0.2) (layer "F.Cu") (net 24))
 (segment (start 145 65) (end 144.536 64.536) (width 0.2) (layer "F.Cu") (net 24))
 (segment (start 155.75 63.965) (end 154.3925 62.6075) (width 0.2) (layer "F.Cu") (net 24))
 (segment (start 143.172 64.536) (end 144.536 64.536) (width 0.2) (layer "F.Cu") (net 24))
 (segment (start 155.75 64.79) (end 155.75 63.965) (width 0.2) (layer "F.Cu") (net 24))
 (via (at 153 64) (size 0.6) (drill 0.3) (layers "F.Cu" "B.Cu") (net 24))
 (via (at 145 65) (size 0.6) (drill 0.3) (layers "F.Cu" "B.Cu") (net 24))
 (segment (start 153 64) (end 146 64) (width 0.2) (layer "B.Cu") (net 24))
 (segment (start 146 64) (end 145 65) (width 0.2) (layer "B.Cu") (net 24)))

